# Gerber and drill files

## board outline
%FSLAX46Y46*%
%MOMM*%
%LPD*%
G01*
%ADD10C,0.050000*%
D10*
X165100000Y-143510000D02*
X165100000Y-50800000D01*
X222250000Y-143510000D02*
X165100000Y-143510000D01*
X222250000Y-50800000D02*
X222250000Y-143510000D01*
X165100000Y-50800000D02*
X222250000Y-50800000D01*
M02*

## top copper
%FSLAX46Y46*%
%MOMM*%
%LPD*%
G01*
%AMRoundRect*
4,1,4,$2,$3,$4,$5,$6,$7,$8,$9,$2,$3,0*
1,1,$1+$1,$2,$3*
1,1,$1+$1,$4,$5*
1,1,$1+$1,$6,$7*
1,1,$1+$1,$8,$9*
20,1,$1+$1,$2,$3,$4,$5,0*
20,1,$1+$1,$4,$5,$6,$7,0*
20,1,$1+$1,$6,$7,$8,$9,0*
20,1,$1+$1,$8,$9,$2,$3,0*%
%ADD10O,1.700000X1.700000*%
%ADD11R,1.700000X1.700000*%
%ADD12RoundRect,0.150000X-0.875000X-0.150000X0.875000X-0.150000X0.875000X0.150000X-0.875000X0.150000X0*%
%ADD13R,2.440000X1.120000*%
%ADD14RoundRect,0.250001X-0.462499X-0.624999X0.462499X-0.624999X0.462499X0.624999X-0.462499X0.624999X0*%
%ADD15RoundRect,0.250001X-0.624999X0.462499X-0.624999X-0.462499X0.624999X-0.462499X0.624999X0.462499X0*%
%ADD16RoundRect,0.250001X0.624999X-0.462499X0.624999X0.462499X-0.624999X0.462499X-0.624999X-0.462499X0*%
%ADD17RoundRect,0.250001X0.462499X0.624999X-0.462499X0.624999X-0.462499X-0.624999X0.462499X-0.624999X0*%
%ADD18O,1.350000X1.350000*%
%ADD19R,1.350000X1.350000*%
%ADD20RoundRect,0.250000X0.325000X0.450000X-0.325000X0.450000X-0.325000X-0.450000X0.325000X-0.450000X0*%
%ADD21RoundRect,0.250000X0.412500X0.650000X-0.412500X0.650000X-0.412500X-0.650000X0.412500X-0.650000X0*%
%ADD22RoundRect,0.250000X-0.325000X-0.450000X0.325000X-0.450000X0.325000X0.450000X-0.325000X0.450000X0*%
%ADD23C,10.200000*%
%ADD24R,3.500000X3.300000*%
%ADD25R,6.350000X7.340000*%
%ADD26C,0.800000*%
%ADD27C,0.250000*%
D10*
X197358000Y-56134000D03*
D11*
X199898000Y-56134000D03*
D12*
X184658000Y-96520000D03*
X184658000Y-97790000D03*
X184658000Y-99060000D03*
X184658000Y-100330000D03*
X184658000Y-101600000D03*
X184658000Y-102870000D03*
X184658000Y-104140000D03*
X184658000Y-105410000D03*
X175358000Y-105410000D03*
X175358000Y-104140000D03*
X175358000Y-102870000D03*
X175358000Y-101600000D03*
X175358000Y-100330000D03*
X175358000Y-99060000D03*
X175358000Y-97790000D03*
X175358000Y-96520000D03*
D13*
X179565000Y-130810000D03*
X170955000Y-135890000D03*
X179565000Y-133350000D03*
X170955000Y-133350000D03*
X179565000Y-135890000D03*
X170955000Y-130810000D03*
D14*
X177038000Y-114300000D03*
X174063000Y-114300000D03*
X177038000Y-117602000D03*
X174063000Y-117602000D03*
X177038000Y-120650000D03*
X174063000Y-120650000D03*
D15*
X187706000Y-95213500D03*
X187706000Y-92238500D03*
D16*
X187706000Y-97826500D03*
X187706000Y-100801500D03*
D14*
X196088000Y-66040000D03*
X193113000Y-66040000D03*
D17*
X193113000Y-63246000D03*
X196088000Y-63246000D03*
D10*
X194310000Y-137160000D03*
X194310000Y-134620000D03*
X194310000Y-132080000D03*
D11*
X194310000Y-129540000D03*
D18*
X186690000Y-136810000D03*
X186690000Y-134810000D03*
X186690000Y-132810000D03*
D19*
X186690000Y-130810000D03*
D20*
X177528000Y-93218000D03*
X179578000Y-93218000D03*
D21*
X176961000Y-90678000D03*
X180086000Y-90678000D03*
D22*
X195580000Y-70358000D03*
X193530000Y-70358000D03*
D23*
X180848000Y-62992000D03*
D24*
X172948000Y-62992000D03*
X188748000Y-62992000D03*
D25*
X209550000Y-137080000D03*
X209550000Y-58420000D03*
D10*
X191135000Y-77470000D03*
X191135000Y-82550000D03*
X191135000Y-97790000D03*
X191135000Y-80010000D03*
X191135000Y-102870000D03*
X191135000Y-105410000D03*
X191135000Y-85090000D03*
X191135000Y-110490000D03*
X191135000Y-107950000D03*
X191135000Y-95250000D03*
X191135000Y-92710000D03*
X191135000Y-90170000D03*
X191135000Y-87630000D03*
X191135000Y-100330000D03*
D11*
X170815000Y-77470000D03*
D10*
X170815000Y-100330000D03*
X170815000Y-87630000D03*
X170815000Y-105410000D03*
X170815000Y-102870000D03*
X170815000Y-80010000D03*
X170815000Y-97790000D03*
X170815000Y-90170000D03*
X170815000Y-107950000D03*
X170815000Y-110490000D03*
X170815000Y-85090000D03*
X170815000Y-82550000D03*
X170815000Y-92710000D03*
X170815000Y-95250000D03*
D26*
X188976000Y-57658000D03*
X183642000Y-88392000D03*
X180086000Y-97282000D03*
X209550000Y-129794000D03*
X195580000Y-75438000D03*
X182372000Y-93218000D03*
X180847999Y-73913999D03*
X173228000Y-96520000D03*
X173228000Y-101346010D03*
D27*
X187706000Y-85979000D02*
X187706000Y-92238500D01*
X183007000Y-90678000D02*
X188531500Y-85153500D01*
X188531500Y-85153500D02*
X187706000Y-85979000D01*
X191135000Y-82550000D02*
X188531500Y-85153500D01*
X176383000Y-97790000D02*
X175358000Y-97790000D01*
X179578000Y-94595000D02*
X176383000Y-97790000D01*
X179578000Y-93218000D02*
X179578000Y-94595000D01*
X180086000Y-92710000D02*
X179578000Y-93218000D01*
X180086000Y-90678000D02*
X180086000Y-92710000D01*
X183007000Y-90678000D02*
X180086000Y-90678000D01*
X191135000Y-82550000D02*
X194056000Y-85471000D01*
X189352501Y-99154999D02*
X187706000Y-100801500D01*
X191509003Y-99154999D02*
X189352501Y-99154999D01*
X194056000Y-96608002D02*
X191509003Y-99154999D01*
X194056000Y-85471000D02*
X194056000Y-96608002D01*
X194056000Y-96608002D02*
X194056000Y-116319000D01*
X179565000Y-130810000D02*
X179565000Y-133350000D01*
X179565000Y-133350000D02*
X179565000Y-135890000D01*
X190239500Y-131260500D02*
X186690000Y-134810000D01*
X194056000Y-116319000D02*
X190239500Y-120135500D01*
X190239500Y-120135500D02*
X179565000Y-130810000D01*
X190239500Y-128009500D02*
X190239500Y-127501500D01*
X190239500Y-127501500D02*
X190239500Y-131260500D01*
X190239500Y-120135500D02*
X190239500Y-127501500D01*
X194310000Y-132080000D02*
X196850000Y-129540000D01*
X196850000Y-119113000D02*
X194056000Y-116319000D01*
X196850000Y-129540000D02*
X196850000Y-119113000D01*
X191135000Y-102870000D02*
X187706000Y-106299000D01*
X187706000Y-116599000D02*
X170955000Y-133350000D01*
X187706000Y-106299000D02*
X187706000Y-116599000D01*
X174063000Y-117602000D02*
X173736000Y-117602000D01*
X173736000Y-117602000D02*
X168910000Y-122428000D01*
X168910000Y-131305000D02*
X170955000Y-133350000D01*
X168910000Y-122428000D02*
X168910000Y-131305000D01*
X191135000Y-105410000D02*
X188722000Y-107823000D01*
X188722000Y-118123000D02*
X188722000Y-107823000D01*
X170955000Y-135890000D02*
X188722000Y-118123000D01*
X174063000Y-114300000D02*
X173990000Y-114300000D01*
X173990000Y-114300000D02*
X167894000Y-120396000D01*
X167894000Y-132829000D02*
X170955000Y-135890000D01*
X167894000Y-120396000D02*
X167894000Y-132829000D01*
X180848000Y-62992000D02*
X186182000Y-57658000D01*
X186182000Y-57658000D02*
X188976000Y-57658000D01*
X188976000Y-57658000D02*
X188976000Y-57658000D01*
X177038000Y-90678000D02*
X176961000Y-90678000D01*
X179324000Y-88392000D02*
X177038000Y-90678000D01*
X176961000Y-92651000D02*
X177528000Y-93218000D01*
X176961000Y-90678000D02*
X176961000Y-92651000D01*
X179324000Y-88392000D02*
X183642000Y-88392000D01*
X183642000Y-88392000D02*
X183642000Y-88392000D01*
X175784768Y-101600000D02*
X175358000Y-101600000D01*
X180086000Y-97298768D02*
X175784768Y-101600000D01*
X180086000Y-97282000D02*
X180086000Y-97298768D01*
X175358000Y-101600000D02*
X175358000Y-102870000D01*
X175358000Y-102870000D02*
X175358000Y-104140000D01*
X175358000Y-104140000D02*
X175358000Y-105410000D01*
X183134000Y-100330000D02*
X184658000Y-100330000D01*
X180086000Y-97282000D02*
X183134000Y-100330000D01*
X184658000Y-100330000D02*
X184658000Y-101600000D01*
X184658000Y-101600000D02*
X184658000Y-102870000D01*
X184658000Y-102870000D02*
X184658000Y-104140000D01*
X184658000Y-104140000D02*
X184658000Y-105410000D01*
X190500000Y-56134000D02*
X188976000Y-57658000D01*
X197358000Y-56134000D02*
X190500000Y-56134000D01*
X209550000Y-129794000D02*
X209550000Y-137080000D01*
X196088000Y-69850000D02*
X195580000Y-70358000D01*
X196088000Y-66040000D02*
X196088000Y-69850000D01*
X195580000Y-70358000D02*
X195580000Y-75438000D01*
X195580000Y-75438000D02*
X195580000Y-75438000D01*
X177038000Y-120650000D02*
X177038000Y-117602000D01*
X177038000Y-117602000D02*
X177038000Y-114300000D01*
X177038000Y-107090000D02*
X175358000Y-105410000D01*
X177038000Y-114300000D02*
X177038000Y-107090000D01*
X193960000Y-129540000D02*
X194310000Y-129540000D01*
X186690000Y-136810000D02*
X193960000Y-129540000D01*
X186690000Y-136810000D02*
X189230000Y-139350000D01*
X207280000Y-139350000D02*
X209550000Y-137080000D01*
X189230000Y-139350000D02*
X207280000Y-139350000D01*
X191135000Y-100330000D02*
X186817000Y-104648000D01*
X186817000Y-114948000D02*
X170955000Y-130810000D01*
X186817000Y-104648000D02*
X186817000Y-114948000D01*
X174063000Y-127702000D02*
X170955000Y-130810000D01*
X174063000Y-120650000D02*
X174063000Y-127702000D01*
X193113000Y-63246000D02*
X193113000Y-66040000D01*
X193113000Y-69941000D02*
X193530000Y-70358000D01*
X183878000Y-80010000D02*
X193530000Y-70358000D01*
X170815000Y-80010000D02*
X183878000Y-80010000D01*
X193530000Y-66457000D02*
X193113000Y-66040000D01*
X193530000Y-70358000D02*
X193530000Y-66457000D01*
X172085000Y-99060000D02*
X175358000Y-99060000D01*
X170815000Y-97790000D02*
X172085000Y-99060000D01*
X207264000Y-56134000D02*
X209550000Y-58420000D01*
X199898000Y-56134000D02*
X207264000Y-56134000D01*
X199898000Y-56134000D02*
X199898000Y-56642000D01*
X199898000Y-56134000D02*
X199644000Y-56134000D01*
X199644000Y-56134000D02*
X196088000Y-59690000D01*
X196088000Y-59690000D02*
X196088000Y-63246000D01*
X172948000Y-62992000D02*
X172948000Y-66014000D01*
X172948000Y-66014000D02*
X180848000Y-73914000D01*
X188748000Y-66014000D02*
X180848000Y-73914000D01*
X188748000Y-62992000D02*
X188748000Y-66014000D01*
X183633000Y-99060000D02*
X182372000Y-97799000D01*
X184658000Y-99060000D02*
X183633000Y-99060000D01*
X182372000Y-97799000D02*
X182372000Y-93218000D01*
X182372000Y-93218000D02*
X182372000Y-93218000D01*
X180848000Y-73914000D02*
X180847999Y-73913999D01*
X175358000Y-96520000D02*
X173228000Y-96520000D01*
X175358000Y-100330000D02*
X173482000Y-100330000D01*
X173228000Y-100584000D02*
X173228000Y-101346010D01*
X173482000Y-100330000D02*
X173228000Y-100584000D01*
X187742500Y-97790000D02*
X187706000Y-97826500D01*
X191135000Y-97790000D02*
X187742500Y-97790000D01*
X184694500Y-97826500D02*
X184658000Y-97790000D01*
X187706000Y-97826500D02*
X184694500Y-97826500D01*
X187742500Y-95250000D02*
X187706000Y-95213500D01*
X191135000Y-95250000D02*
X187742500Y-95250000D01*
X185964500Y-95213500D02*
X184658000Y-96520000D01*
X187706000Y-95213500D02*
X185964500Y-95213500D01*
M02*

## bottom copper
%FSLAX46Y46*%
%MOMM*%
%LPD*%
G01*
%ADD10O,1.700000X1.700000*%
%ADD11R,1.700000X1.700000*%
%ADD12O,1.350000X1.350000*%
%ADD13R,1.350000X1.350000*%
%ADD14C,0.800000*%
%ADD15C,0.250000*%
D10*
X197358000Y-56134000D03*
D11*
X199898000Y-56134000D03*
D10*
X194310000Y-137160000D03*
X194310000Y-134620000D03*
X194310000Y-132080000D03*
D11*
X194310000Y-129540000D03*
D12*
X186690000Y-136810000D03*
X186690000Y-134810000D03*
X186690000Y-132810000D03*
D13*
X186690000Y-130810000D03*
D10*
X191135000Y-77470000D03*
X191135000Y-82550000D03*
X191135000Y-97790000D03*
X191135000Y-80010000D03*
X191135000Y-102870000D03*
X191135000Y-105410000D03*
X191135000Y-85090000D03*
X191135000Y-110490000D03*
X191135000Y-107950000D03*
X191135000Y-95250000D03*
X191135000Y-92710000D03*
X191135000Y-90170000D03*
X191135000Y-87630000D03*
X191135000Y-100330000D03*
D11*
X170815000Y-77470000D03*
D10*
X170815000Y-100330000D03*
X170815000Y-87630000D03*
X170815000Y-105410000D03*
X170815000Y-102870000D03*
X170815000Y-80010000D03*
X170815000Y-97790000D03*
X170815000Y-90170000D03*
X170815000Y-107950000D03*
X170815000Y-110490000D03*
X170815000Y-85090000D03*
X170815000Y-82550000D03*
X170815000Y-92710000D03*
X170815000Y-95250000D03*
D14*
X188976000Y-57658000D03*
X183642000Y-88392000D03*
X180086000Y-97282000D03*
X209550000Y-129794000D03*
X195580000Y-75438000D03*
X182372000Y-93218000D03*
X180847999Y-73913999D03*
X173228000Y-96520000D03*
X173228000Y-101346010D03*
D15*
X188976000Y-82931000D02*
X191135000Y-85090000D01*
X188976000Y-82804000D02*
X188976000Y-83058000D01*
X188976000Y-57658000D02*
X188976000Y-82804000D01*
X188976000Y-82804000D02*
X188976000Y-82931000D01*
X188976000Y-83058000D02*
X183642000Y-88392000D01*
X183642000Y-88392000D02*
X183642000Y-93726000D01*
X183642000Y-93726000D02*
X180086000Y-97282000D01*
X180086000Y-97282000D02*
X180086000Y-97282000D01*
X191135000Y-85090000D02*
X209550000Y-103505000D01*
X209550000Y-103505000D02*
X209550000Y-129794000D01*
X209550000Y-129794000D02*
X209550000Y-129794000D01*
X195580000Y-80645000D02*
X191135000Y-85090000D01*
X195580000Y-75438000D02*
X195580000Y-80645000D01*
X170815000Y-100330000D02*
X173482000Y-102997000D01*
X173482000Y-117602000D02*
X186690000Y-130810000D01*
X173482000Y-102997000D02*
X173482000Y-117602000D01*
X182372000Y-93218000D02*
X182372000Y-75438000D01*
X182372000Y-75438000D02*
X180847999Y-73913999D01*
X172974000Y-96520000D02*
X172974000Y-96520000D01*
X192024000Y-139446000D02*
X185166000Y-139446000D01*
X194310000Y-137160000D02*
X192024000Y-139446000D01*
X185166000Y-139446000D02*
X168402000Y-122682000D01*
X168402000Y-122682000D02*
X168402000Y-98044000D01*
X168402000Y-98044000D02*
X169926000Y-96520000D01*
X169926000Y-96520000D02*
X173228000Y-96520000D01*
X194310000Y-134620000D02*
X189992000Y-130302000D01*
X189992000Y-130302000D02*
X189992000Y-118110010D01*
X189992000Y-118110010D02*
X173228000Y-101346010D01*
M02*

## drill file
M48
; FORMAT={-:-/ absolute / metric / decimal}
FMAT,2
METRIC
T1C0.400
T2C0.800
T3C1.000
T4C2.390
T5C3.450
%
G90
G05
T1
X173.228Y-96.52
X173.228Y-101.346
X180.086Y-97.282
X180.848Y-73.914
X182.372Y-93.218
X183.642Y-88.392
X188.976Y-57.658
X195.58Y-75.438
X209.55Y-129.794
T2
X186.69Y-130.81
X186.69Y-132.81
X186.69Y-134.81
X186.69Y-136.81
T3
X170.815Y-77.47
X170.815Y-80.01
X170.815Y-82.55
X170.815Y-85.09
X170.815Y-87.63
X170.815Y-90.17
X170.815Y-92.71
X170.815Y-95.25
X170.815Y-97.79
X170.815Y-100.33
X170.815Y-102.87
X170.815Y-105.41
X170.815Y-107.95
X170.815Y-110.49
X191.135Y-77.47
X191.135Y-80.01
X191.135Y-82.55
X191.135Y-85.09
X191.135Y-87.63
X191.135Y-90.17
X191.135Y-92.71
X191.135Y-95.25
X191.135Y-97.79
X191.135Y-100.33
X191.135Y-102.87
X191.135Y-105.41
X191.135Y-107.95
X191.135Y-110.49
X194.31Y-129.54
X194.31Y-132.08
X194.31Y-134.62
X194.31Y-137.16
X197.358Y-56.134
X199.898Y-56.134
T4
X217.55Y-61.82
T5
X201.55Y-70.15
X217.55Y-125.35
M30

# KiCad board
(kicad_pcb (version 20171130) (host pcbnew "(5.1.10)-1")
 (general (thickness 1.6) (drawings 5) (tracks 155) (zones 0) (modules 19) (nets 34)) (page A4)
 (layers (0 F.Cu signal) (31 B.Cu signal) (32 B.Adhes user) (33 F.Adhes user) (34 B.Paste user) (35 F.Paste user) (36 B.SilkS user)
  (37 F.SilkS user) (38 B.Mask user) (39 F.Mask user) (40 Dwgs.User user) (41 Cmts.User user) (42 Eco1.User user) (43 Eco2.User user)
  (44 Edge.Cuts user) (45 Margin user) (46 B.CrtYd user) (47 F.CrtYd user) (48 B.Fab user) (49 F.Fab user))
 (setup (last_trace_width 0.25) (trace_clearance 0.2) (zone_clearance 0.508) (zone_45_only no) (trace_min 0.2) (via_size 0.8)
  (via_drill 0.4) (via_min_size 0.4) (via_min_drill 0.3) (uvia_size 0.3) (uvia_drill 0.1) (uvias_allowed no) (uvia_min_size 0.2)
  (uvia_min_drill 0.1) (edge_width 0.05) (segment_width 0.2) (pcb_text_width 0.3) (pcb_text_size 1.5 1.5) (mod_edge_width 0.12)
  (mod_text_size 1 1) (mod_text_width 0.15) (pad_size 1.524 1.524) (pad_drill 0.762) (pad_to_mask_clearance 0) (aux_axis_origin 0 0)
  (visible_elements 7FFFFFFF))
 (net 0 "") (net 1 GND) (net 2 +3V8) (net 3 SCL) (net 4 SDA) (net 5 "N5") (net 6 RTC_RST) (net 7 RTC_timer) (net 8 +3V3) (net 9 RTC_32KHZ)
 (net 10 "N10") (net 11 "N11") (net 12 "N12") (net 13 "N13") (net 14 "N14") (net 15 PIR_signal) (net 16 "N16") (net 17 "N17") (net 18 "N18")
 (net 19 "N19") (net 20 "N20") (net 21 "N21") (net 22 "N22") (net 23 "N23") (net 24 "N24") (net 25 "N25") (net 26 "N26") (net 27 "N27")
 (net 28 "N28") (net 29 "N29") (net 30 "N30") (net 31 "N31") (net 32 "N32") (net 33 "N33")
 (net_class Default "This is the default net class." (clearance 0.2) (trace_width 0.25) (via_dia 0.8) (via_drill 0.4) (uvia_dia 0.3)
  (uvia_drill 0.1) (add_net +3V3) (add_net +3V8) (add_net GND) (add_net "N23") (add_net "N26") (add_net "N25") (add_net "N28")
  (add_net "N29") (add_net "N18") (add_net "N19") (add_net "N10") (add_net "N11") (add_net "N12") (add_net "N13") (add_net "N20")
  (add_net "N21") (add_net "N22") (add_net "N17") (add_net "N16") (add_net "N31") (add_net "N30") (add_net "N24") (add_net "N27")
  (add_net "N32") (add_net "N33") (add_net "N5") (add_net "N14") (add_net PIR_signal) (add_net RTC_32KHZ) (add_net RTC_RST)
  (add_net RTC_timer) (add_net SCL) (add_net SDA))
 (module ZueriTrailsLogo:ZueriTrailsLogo (layer B.Cu) (at 201.93 96.52 270)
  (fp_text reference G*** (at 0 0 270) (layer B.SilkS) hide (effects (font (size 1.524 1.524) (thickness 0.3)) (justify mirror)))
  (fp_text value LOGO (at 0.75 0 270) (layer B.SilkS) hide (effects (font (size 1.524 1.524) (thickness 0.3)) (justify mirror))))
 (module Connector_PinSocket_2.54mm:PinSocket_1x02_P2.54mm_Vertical (layer F.Cu) (at 199.898 56.134 270)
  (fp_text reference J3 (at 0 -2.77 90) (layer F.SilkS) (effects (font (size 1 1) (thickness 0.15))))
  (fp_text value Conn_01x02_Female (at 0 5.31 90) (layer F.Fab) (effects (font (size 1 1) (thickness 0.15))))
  (pad 2 thru_hole oval (at 0 2.54 270) (size 1.7 1.7) (drill 1) (layers *.Cu *.Mask) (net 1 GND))
  (pad 1 thru_hole rect (at 0 0 270) (size 1.7 1.7) (drill 1) (layers *.Cu *.Mask) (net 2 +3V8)))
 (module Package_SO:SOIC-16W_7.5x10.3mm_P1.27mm (layer F.Cu) (at 180.008 100.965)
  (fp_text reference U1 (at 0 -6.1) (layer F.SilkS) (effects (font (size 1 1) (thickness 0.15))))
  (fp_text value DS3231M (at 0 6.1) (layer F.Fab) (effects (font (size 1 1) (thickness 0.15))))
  (pad 16 smd roundrect (at 4.65 -4.445) (size 2.05 0.6) (layers F.Cu F.Paste F.Mask) (roundrect_rratio 0.25) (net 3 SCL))
  (pad 15 smd roundrect (at 4.65 -3.175) (size 2.05 0.6) (layers F.Cu F.Paste F.Mask) (roundrect_rratio 0.25) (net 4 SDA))
  (pad 14 smd roundrect (at 4.65 -1.905) (size 2.05 0.6) (layers F.Cu F.Paste F.Mask) (roundrect_rratio 0.25) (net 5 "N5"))
  (pad 13 smd roundrect (at 4.65 -0.635) (size 2.05 0.6) (layers F.Cu F.Paste F.Mask) (roundrect_rratio 0.25) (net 1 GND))
  (pad 12 smd roundrect (at 4.65 0.635) (size 2.05 0.6) (layers F.Cu F.Paste F.Mask) (roundrect_rratio 0.25) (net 1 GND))
  (pad 11 smd roundrect (at 4.65 1.905) (size 2.05 0.6) (layers F.Cu F.Paste F.Mask) (roundrect_rratio 0.25) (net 1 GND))
  (pad 10 smd roundrect (at 4.65 3.175) (size 2.05 0.6) (layers F.Cu F.Paste F.Mask) (roundrect_rratio 0.25) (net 1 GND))
  (pad 9 smd roundrect (at 4.65 4.445) (size 2.05 0.6) (layers F.Cu F.Paste F.Mask) (roundrect_rratio 0.25) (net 1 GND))
  (pad 8 smd roundrect (at -4.65 4.445) (size 2.05 0.6) (layers F.Cu F.Paste F.Mask) (roundrect_rratio 0.25) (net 1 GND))
  (pad 7 smd roundrect (at -4.65 3.175) (size 2.05 0.6) (layers F.Cu F.Paste F.Mask) (roundrect_rratio 0.25) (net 1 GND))
  (pad 6 smd roundrect (at -4.65 1.905) (size 2.05 0.6) (layers F.Cu F.Paste F.Mask) (roundrect_rratio 0.25) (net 1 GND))
  (pad 5 smd roundrect (at -4.65 0.635) (size 2.05 0.6) (layers F.Cu F.Paste F.Mask) (roundrect_rratio 0.25) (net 1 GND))
  (pad 4 smd roundrect (at -4.65 -0.635) (size 2.05 0.6) (layers F.Cu F.Paste F.Mask) (roundrect_rratio 0.25) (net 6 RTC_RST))
  (pad 3 smd roundrect (at -4.65 -1.905) (size 2.05 0.6) (layers F.Cu F.Paste F.Mask) (roundrect_rratio 0.25) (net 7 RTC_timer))
  (pad 2 smd roundrect (at -4.65 -3.175) (size 2.05 0.6) (layers F.Cu F.Paste F.Mask) (roundrect_rratio 0.25) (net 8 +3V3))
  (pad 1 smd roundrect (at -4.65 -4.445) (size 2.05 0.6) (layers F.Cu F.Paste F.Mask) (roundrect_rratio 0.25) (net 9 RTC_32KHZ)))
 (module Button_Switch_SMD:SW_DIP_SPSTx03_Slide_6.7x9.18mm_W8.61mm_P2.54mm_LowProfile (layer F.Cu) (at 175.26 133.35)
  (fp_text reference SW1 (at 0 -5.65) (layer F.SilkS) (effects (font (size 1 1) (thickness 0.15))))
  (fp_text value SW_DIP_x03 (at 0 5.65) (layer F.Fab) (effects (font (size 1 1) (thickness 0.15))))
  (pad 6 smd rect (at 4.305 -2.54) (size 2.44 1.12) (layers F.Cu F.Paste F.Mask) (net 8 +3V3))
  (pad 3 smd rect (at -4.305 2.54) (size 2.44 1.12) (layers F.Cu F.Paste F.Mask) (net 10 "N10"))
  (pad 5 smd rect (at 4.305 0) (size 2.44 1.12) (layers F.Cu F.Paste F.Mask) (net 8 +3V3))
  (pad 2 smd rect (at -4.305 0) (size 2.44 1.12) (layers F.Cu F.Paste F.Mask) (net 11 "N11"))
  (pad 4 smd rect (at 4.305 2.54) (size 2.44 1.12) (layers F.Cu F.Paste F.Mask) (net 8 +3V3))
  (pad 1 smd rect (at -4.305 -2.54) (size 2.44 1.12) (layers F.Cu F.Paste F.Mask) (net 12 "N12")))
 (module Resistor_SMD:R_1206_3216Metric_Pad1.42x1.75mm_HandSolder (layer F.Cu) (at 175.5505 114.3)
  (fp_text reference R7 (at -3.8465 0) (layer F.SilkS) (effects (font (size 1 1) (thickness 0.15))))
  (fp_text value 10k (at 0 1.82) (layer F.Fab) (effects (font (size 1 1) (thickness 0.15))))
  (pad 2 smd roundrect (at 1.4875 0) (size 1.425 1.75) (layers F.Cu F.Paste F.Mask) (roundrect_rratio 0.175439) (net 1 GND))
  (pad 1 smd roundrect (at -1.4875 0) (size 1.425 1.75) (layers F.Cu F.Paste F.Mask) (roundrect_rratio 0.175439) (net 10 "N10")))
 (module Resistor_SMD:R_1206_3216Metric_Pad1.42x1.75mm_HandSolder (layer F.Cu) (at 175.5505 117.602)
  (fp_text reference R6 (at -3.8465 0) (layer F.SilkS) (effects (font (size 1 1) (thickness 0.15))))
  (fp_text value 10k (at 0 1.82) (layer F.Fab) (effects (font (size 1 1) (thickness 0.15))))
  (pad 2 smd roundrect (at 1.4875 0) (size 1.425 1.75) (layers F.Cu F.Paste F.Mask) (roundrect_rratio 0.175439) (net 1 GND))
  (pad 1 smd roundrect (at -1.4875 0) (size 1.425 1.75) (layers F.Cu F.Paste F.Mask) (roundrect_rratio 0.175439) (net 11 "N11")))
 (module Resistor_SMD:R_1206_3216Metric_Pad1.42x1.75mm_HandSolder (layer F.Cu) (at 175.5505 120.65)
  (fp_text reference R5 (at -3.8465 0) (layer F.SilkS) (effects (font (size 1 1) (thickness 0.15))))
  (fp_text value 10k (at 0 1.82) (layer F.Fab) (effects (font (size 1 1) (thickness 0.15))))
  (pad 2 smd roundrect (at 1.4875 0) (size 1.425 1.75) (layers F.Cu F.Paste F.Mask) (roundrect_rratio 0.175439) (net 1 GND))
  (pad 1 smd roundrect (at -1.4875 0) (size 1.425 1.75) (layers F.Cu F.Paste F.Mask) (roundrect_rratio 0.175439) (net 12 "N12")))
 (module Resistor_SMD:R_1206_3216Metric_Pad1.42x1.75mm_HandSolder (layer F.Cu) (at 187.706 93.726 270)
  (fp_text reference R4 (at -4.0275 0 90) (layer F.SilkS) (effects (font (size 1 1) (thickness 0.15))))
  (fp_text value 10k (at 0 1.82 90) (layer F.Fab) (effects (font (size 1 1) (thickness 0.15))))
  (pad 2 smd roundrect (at 1.4875 0 270) (size 1.425 1.75) (layers F.Cu F.Paste F.Mask) (roundrect_rratio 0.175439) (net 3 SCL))
  (pad 1 smd roundrect (at -1.4875 0 270) (size 1.425 1.75) (layers F.Cu F.Paste F.Mask) (roundrect_rratio 0.175439) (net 8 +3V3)))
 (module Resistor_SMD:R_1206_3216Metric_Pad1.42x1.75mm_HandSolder (layer F.Cu) (at 187.706 99.314 90)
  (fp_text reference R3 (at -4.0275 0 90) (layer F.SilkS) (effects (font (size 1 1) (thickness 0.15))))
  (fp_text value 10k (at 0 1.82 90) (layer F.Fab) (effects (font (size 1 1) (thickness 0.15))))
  (pad 2 smd roundrect (at 1.4875 0 90) (size 1.425 1.75) (layers F.Cu F.Paste F.Mask) (roundrect_rratio 0.175439) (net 4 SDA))
  (pad 1 smd roundrect (at -1.4875 0 90) (size 1.425 1.75) (layers F.Cu F.Paste F.Mask) (roundrect_rratio 0.175439) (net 8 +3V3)))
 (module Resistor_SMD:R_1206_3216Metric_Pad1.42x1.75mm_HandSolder (layer F.Cu) (at 194.6005 66.04)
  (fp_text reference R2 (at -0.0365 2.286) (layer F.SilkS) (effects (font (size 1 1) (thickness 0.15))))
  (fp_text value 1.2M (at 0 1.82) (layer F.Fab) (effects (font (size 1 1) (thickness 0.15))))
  (pad 2 smd roundrect (at 1.4875 0) (size 1.425 1.75) (layers F.Cu F.Paste F.Mask) (roundrect_rratio 0.175439) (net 1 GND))
  (pad 1 smd roundrect (at -1.4875 0) (size 1.425 1.75) (layers F.Cu F.Paste F.Mask) (roundrect_rratio 0.175439) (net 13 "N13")))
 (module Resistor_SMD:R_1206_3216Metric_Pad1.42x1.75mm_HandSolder (layer F.Cu) (at 194.6005 63.246 180)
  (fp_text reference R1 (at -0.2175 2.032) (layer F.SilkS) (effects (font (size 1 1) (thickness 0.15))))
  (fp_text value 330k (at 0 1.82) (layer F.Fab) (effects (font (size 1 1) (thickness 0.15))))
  (pad 2 smd roundrect (at 1.4875 0 180) (size 1.425 1.75) (layers F.Cu F.Paste F.Mask) (roundrect_rratio 0.175439) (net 13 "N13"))
  (pad 1 smd roundrect (at -1.4875 0 180) (size 1.425 1.75) (layers F.Cu F.Paste F.Mask) (roundrect_rratio 0.175439) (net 2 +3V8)))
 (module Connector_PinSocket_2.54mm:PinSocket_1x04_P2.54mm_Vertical (layer F.Cu) (at 194.31 129.54)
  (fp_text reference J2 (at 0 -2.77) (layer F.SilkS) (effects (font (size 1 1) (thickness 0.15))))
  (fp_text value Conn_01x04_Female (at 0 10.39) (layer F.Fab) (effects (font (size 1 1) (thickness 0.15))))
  (pad 4 thru_hole oval (at 0 7.62) (size 1.7 1.7) (drill 1) (layers *.Cu *.Mask) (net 9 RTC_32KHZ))
  (pad 3 thru_hole oval (at 0 5.08) (size 1.7 1.7) (drill 1) (layers *.Cu *.Mask) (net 6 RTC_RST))
  (pad 2 thru_hole oval (at 0 2.54) (size 1.7 1.7) (drill 1) (layers *.Cu *.Mask) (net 8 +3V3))
  (pad 1 thru_hole rect (at 0 0) (size 1.7 1.7) (drill 1) (layers *.Cu *.Mask) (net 1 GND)))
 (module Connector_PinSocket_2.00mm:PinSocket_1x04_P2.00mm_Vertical (layer F.Cu) (at 186.69 130.81)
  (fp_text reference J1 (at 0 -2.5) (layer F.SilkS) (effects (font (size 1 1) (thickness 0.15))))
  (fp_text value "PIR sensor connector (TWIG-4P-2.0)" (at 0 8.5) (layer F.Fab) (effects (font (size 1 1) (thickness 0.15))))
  (pad 4 thru_hole oval (at 0 6) (size 1.35 1.35) (drill 0.8) (layers *.Cu *.Mask) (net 1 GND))
  (pad 3 thru_hole oval (at 0 4) (size 1.35 1.35) (drill 0.8) (layers *.Cu *.Mask) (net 8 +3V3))
  (pad 2 thru_hole oval (at 0 2) (size 1.35 1.35) (drill 0.8) (layers *.Cu *.Mask) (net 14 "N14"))
  (pad 1 thru_hole rect (at 0 0) (size 1.35 1.35) (drill 0.8) (layers *.Cu *.Mask) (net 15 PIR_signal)))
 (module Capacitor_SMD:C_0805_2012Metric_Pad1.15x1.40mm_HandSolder (layer F.Cu) (at 178.553 93.218 180)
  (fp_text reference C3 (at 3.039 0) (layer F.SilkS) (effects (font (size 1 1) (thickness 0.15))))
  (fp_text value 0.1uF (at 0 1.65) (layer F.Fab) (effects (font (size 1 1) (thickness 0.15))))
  (pad 2 smd roundrect (at 1.025 0 180) (size 1.15 1.4) (layers F.Cu F.Paste F.Mask) (roundrect_rratio 0.217391) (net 1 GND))
  (pad 1 smd roundrect (at -1.025 0 180) (size 1.15 1.4) (layers F.Cu F.Paste F.Mask) (roundrect_rratio 0.217391) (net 8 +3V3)))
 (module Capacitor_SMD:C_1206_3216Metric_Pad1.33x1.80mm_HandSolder (layer F.Cu) (at 178.5235 90.678 180)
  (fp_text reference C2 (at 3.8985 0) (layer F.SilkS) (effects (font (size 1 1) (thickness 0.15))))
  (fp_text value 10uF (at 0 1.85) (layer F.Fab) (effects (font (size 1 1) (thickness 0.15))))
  (pad 2 smd roundrect (at 1.5625 0 180) (size 1.325 1.8) (layers F.Cu F.Paste F.Mask) (roundrect_rratio 0.188679) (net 1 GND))
  (pad 1 smd roundrect (at -1.5625 0 180) (size 1.325 1.8) (layers F.Cu F.Paste F.Mask) (roundrect_rratio 0.188679) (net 8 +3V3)))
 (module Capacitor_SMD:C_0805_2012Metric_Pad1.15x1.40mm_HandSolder (layer F.Cu) (at 194.555 70.358)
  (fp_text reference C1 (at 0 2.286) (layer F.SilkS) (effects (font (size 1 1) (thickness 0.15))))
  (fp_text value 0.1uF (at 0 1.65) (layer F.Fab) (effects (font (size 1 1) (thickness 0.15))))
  (pad 2 smd roundrect (at 1.025 0) (size 1.15 1.4) (layers F.Cu F.Paste F.Mask) (roundrect_rratio 0.217391) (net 1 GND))
  (pad 1 smd roundrect (at -1.025 0) (size 1.15 1.4) (layers F.Cu F.Paste F.Mask) (roundrect_rratio 0.217391) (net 13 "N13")))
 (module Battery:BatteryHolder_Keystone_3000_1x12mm (layer F.Cu) (at 180.848 62.992 180)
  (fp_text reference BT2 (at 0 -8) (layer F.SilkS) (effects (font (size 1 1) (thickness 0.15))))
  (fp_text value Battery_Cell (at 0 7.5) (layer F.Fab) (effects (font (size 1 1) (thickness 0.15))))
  (pad 2 smd circle (at 0 0 180) (size 10.2 10.2) (layers F.Cu F.Mask) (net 1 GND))
  (pad 1 smd rect (at 7.9 0 180) (size 3.5 3.3) (layers F.Cu F.Paste F.Mask) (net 5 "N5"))
  (pad 1 smd rect (at -7.9 0 180) (size 3.5 3.3) (layers F.Cu F.Paste F.Mask) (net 5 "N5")))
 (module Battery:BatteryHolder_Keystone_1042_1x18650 (layer F.Cu) (at 209.55 97.75 270)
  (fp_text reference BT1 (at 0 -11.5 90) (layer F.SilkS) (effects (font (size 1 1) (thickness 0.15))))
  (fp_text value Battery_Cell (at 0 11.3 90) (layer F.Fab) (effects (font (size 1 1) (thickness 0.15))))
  (pad "" np_thru_hole circle (at -35.93 -8 270) (size 2.39 2.39) (drill 2.39) (layers *.Cu *.Mask))
  (pad "" np_thru_hole circle (at -27.6 8 270) (size 3.45 3.45) (drill 3.45) (layers *.Cu *.Mask))
  (pad "" np_thru_hole circle (at 27.6 -8 270) (size 3.45 3.45) (drill 3.45) (layers *.Cu *.Mask))
  (pad 2 smd rect (at 39.33 0 270) (size 7.34 6.35) (layers F.Cu F.Paste F.Mask) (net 1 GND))
  (pad 1 smd rect (at -39.33 0 270) (size 7.34 6.35) (layers F.Cu F.Paste F.Mask) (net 2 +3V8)))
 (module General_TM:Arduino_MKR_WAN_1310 (layer F.Cu) (at 170.815 77.47)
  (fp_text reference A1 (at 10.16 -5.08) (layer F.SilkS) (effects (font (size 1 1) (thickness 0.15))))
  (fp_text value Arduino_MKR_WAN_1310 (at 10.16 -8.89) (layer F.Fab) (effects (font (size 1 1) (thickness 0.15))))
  (pad 28 thru_hole oval (at 20.32 0) (size 1.7 1.7) (drill 1) (layers *.Cu *.Mask) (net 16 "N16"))
  (pad 26 thru_hole oval (at 20.32 5.08) (size 1.7 1.7) (drill 1) (layers *.Cu *.Mask) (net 8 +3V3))
  (pad 20 thru_hole oval (at 20.32 20.32) (size 1.7 1.7) (drill 1) (layers *.Cu *.Mask) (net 4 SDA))
  (pad 27 thru_hole oval (at 20.32 2.54) (size 1.7 1.7) (drill 1) (layers *.Cu *.Mask) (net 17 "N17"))
  (pad 18 thru_hole oval (at 20.32 25.4) (size 1.7 1.7) (drill 1) (layers *.Cu *.Mask) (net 11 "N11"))
  (pad 17 thru_hole oval (at 20.32 27.94) (size 1.7 1.7) (drill 1) (layers *.Cu *.Mask) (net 10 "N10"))
  (pad 25 thru_hole oval (at 20.32 7.62) (size 1.7 1.7) (drill 1) (layers *.Cu *.Mask) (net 1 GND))
  (pad 15 thru_hole oval (at 20.32 33.02) (size 1.7 1.7) (drill 1) (layers *.Cu *.Mask) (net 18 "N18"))
  (pad 16 thru_hole oval (at 20.32 30.48) (size 1.7 1.7) (drill 1) (layers *.Cu *.Mask) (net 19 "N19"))
  (pad 21 thru_hole oval (at 20.32 17.78) (size 1.7 1.7) (drill 1) (layers *.Cu *.Mask) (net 3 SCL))
  (pad 22 thru_hole oval (at 20.32 15.24) (size 1.7 1.7) (drill 1) (layers *.Cu *.Mask) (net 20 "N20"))
  (pad 23 thru_hole oval (at 20.32 12.7) (size 1.7 1.7) (drill 1) (layers *.Cu *.Mask) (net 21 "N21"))
  (pad 24 thru_hole oval (at 20.32 10.16) (size 1.7 1.7) (drill 1) (layers *.Cu *.Mask) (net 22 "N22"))
  (pad 19 thru_hole oval (at 20.32 22.86) (size 1.7 1.7) (drill 1) (layers *.Cu *.Mask) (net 12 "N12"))
  (pad 1 thru_hole rect (at 0 0) (size 1.7 1.7) (drill 1) (layers *.Cu *.Mask) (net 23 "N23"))
  (pad 10 thru_hole oval (at 0 22.86) (size 1.7 1.7) (drill 1) (layers *.Cu *.Mask) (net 15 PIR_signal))
  (pad 5 thru_hole oval (at 0 10.16) (size 1.7 1.7) (drill 1) (layers *.Cu *.Mask) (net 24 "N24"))
  (pad 12 thru_hole oval (at 0 27.94) (size 1.7 1.7) (drill 1) (layers *.Cu *.Mask) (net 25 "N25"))
  (pad 11 thru_hole oval (at 0 25.4) (size 1.7 1.7) (drill 1) (layers *.Cu *.Mask) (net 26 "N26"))
  (pad 2 thru_hole oval (at 0 2.54) (size 1.7 1.7) (drill 1) (layers *.Cu *.Mask) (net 13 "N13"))
  (pad 9 thru_hole oval (at 0 20.32) (size 1.7 1.7) (drill 1) (layers *.Cu *.Mask) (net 7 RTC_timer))
  (pad 6 thru_hole oval (at 0 12.7) (size 1.7 1.7) (drill 1) (layers *.Cu *.Mask) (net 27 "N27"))
  (pad 13 thru_hole oval (at 0 30.48) (size 1.7 1.7) (drill 1) (layers *.Cu *.Mask) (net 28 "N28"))
  (pad 14 thru_hole oval (at 0 33.02) (size 1.7 1.7) (drill 1) (layers *.Cu *.Mask) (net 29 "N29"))
  (pad 4 thru_hole oval (at 0 7.62) (size 1.7 1.7) (drill 1) (layers *.Cu *.Mask) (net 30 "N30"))
  (pad 3 thru_hole oval (at 0 5.08) (size 1.7 1.7) (drill 1) (layers *.Cu *.Mask) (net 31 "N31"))
  (pad 7 thru_hole oval (at 0 15.24) (size 1.7 1.7) (drill 1) (layers *.Cu *.Mask) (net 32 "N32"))
  (pad 8 thru_hole oval (at 0 17.78) (size 1.7 1.7) (drill 1) (layers *.Cu *.Mask) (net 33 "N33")))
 (gr_line (start 165.1 143.51) (end 165.1 50.8) (layer Edge.Cuts) (width 0.05))
 (gr_line (start 222.25 143.51) (end 165.1 143.51) (layer Edge.Cuts) (width 0.05))
 (gr_line (start 222.25 50.8) (end 222.25 143.51) (layer Edge.Cuts) (width 0.05))
 (gr_line (start 165.1 50.8) (end 222.25 50.8) (layer Edge.Cuts) (width 0.05))
 (segment (start 187.706 85.979) (end 187.706 92.2385) (width 0.25) (layer F.Cu) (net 8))
 (segment (start 183.007 90.678) (end 188.5315 85.1535) (width 0.25) (layer F.Cu) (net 8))
 (segment (start 188.5315 85.1535) (end 187.706 85.979) (width 0.25) (layer F.Cu) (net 8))
 (segment (start 191.135 82.55) (end 188.5315 85.1535) (width 0.25) (layer F.Cu) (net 8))
 (segment (start 176.383 97.79) (end 175.358 97.79) (width 0.25) (layer F.Cu) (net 8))
 (segment (start 179.578 94.595) (end 176.383 97.79) (width 0.25) (layer F.Cu) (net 8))
 (segment (start 179.578 93.218) (end 179.578 94.595) (width 0.25) (layer F.Cu) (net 8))
 (segment (start 180.086 92.71) (end 179.578 93.218) (width 0.25) (layer F.Cu) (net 8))
 (segment (start 180.086 90.678) (end 180.086 92.71) (width 0.25) (layer F.Cu) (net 8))
 (segment (start 183.007 90.678) (end 180.086 90.678) (width 0.25) (layer F.Cu) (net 8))
 (segment (start 191.135 82.55) (end 194.056 85.471) (width 0.25) (layer F.Cu) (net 8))
 (segment (start 189.352501 99.154999) (end 187.706 100.8015) (width 0.25) (layer F.Cu) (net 8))
 (segment (start 191.509003 99.154999) (end 189.352501 99.154999) (width 0.25) (layer F.Cu) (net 8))
 (segment (start 194.056 96.608002) (end 191.509003 99.154999) (width 0.25) (layer F.Cu) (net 8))
 (segment (start 194.056 85.471) (end 194.056 96.608002) (width 0.25) (layer F.Cu) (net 8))
 (segment (start 194.056 96.608002) (end 194.056 116.319) (width 0.25) (layer F.Cu) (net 8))
 (segment (start 179.565 130.81) (end 179.565 133.35) (width 0.25) (layer F.Cu) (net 8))
 (segment (start 179.565 133.35) (end 179.565 135.89) (width 0.25) (layer F.Cu) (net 8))
 (segment (start 190.2395 131.2605) (end 186.69 134.81) (width 0.25) (layer F.Cu) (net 8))
 (segment (start 194.056 116.319) (end 190.2395 120.1355) (width 0.25) (layer F.Cu) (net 8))
 (segment (start 190.2395 120.1355) (end 179.565 130.81) (width 0.25) (layer F.Cu) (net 8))
 (segment (start 190.2395 128.0095) (end 190.2395 127.5015) (width 0.25) (layer F.Cu) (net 8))
 (segment (start 190.2395 127.5015) (end 190.2395 131.2605) (width 0.25) (layer F.Cu) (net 8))
 (segment (start 190.2395 120.1355) (end 190.2395 127.5015) (width 0.25) (layer F.Cu) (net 8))
 (segment (start 194.31 132.08) (end 196.85 129.54) (width 0.25) (layer F.Cu) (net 8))
 (segment (start 196.85 119.113) (end 194.056 116.319) (width 0.25) (layer F.Cu) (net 8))
 (segment (start 196.85 129.54) (end 196.85 119.113) (width 0.25) (layer F.Cu) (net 8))
 (segment (start 191.135 102.87) (end 187.706 106.299) (width 0.25) (layer F.Cu) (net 11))
 (segment (start 187.706 116.599) (end 170.955 133.35) (width 0.25) (layer F.Cu) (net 11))
 (segment (start 187.706 106.299) (end 187.706 116.599) (width 0.25) (layer F.Cu) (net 11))
 (segment (start 174.063 117.602) (end 173.736 117.602) (width 0.25) (layer F.Cu) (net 11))
 (segment (start 173.736 117.602) (end 168.91 122.428) (width 0.25) (layer F.Cu) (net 11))
 (segment (start 168.91 131.305) (end 170.955 133.35) (width 0.25) (layer F.Cu) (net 11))
 (segment (start 168.91 122.428) (end 168.91 131.305) (width 0.25) (layer F.Cu) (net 11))
 (segment (start 191.135 105.41) (end 188.722 107.823) (width 0.25) (layer F.Cu) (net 10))
 (segment (start 188.722 118.123) (end 188.722 107.823) (width 0.25) (layer F.Cu) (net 10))
 (segment (start 170.955 135.89) (end 188.722 118.123) (width 0.25) (layer F.Cu) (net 10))
 (segment (start 174.063 114.3) (end 173.99 114.3) (width 0.25) (layer F.Cu) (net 10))
 (segment (start 173.99 114.3) (end 167.894 120.396) (width 0.25) (layer F.Cu) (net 10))
 (segment (start 167.894 132.829) (end 170.955 135.89) (width 0.25) (layer F.Cu) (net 10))
 (segment (start 167.894 120.396) (end 167.894 132.829) (width 0.25) (layer F.Cu) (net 10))
 (segment (start 180.848 62.992) (end 186.182 57.658) (width 0.25) (layer F.Cu) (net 1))
 (segment (start 186.182 57.658) (end 188.976 57.658) (width 0.25) (layer F.Cu) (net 1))
 (segment (start 188.976 57.658) (end 188.976 57.658) (width 0.25) (layer F.Cu) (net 1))
 (via (at 188.976 57.658) (size 0.8) (drill 0.4) (layers F.Cu B.Cu) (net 1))
 (segment (start 188.976 82.931) (end 191.135 85.09) (width 0.25) (layer B.Cu) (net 1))
 (segment (start 188.976 82.804) (end 188.976 83.058) (width 0.25) (layer B.Cu) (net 1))
 (segment (start 188.976 57.658) (end 188.976 82.804) (width 0.25) (layer B.Cu) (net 1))
 (segment (start 188.976 82.804) (end 188.976 82.931) (width 0.25) (layer B.Cu) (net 1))
 (segment (start 188.976 83.058) (end 183.642 88.392) (width 0.25) (layer B.Cu) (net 1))
 (segment (start 177.038 90.678) (end 176.961 90.678) (width 0.25) (layer F.Cu) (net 1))
 (segment (start 179.324 88.392) (end 177.038 90.678) (width 0.25) (layer F.Cu) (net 1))
 (segment (start 176.961 92.651) (end 177.528 93.218) (width 0.25) (layer F.Cu) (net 1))
 (segment (start 176.961 90.678) (end 176.961 92.651) (width 0.25) (layer F.Cu) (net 1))
 (segment (start 179.324 88.392) (end 183.642 88.392) (width 0.25) (layer F.Cu) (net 1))
 (segment (start 183.642 88.392) (end 183.642 88.392) (width 0.25) (layer F.Cu) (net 1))
 (via (at 183.642 88.392) (size 0.8) (drill 0.4) (layers F.Cu B.Cu) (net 1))
 (segment (start 183.642 88.392) (end 183.642 93.726) (width 0.25) (layer B.Cu) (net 1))
 (segment (start 183.642 93.726) (end 180.086 97.282) (width 0.25) (layer B.Cu) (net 1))
 (segment (start 180.086 97.282) (end 180.086 97.282) (width 0.25) (layer B.Cu) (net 1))
 (via (at 180.086 97.282) (size 0.8) (drill 0.4) (layers F.Cu B.Cu) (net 1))
 (segment (start 175.784768 101.6) (end 175.358 101.6) (width 0.25) (layer F.Cu) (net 1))
 (segment (start 180.086 97.298768) (end 175.784768 101.6) (width 0.25) (layer F.Cu) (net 1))
 (segment (start 180.086 97.282) (end 180.086 97.298768) (width 0.25) (layer F.Cu) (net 1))
 (segment (start 175.358 101.6) (end 175.358 102.87) (width 0.25) (layer F.Cu) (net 1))
 (segment (start 175.358 102.87) (end 175.358 104.14) (width 0.25) (layer F.Cu) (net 1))
 (segment (start 175.358 104.14) (end 175.358 105.41) (width 0.25) (layer F.Cu) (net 1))
 (segment (start 183.134 100.33) (end 184.658 100.33) (width 0.25) (layer F.Cu) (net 1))
 (segment (start 180.086 97.282) (end 183.134 100.33) (width 0.25) (layer F.Cu) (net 1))
 (segment (start 184.658 100.33) (end 184.658 101.6) (width 0.25) (layer F.Cu) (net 1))
 (segment (start 184.658 101.6) (end 184.658 102.87) (width 0.25) (layer F.Cu) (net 1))
 (segment (start 184.658 102.87) (end 184.658 104.14) (width 0.25) (layer F.Cu) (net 1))
 (segment (start 184.658 104.14) (end 184.658 105.41) (width 0.25) (layer F.Cu) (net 1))
 (segment (start 190.5 56.134) (end 188.976 57.658) (width 0.25) (layer F.Cu) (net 1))
 (segment (start 197.358 56.134) (end 190.5 56.134) (width 0.25) (layer F.Cu) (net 1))
 (segment (start 191.135 85.09) (end 209.55 103.505) (width 0.25) (layer B.Cu) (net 1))
 (segment (start 209.55 103.505) (end 209.55 129.794) (width 0.25) (layer B.Cu) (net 1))
 (segment (start 209.55 129.794) (end 209.55 129.794) (width 0.25) (layer B.Cu) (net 1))
 (via (at 209.55 129.794) (size 0.8) (drill 0.4) (layers F.Cu B.Cu) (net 1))
 (segment (start 209.55 129.794) (end 209.55 137.08) (width 0.25) (layer F.Cu) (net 1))
 (segment (start 196.088 69.85) (end 195.58 70.358) (width 0.25) (layer F.Cu) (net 1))
 (segment (start 196.088 66.04) (end 196.088 69.85) (width 0.25) (layer F.Cu) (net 1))
 (segment (start 195.58 70.358) (end 195.58 75.438) (width 0.25) (layer F.Cu) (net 1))
 (segment (start 195.58 75.438) (end 195.58 75.438) (width 0.25) (layer F.Cu) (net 1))
 (via (at 195.58 75.438) (size 0.8) (drill 0.4) (layers F.Cu B.Cu) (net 1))
 (segment (start 195.58 80.645) (end 191.135 85.09) (width 0.25) (layer B.Cu) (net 1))
 (segment (start 195.58 75.438) (end 195.58 80.645) (width 0.25) (layer B.Cu) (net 1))
 (segment (start 177.038 120.65) (end 177.038 117.602) (width 0.25) (layer F.Cu) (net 1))
 (segment (start 177.038 117.602) (end 177.038 114.3) (width 0.25) (layer F.Cu) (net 1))
 (segment (start 177.038 107.09) (end 175.358 105.41) (width 0.25) (layer F.Cu) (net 1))
 (segment (start 177.038 114.3) (end 177.038 107.09) (width 0.25) (layer F.Cu) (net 1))
 (segment (start 193.96 129.54) (end 194.31 129.54) (width 0.25) (layer F.Cu) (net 1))
 (segment (start 186.69 136.81) (end 193.96 129.54) (width 0.25) (layer F.Cu) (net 1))
 (segment (start 186.69 136.81) (end 189.23 139.35) (width 0.25) (layer F.Cu) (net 1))
 (segment (start 207.28 139.35) (end 209.55 137.08) (width 0.25) (layer F.Cu) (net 1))
 (segment (start 189.23 139.35) (end 207.28 139.35) (width 0.25) (layer F.Cu) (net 1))
 (segment (start 191.135 100.33) (end 186.817 104.648) (width 0.25) (layer F.Cu) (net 12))
 (segment (start 186.817 114.948) (end 170.955 130.81) (width 0.25) (layer F.Cu) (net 12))
 (segment (start 186.817 104.648) (end 186.817 114.948) (width 0.25) (layer F.Cu) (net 12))
 (segment (start 174.063 127.702) (end 170.955 130.81) (width 0.25) (layer F.Cu) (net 12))
 (segment (start 174.063 120.65) (end 174.063 127.702) (width 0.25) (layer F.Cu) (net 12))
 (segment (start 170.815 100.33) (end 173.482 102.997) (width 0.25) (layer B.Cu) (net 15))
 (segment (start 173.482 117.602) (end 186.69 130.81) (width 0.25) (layer B.Cu) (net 15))
 (segment (start 173.482 102.997) (end 173.482 117.602) (width 0.25) (layer B.Cu) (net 15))
 (segment (start 193.113 63.246) (end 193.113 66.04) (width 0.25) (layer F.Cu) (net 13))
 (segment (start 193.113 69.941) (end 193.53 70.358) (width 0.25) (layer F.Cu) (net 13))
 (segment (start 183.878 80.01) (end 193.53 70.358) (width 0.25) (layer F.Cu) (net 13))
 (segment (start 170.815 80.01) (end 183.878 80.01) (width 0.25) (layer F.Cu) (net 13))
 (segment (start 193.53 66.457) (end 193.113 66.04) (width 0.25) (layer F.Cu) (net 13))
 (segment (start 193.53 70.358) (end 193.53 66.457) (width 0.25) (layer F.Cu) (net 13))
 (segment (start 172.085 99.06) (end 175.358 99.06) (width 0.25) (layer F.Cu) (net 7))
 (segment (start 170.815 97.79) (end 172.085 99.06) (width 0.25) (layer F.Cu) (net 7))
 (segment (start 207.264 56.134) (end 209.55 58.42) (width 0.25) (layer F.Cu) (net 2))
 (segment (start 199.898 56.134) (end 207.264 56.134) (width 0.25) (layer F.Cu) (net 2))
 (segment (start 199.898 56.134) (end 199.898 56.642) (width 0.25) (layer F.Cu) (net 2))
 (segment (start 199.898 56.134) (end 199.644 56.134) (width 0.25) (layer F.Cu) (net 2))
 (segment (start 199.644 56.134) (end 196.088 59.69) (width 0.25) (layer F.Cu) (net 2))
 (segment (start 196.088 59.69) (end 196.088 63.246) (width 0.25) (layer F.Cu) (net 2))
 (segment (start 172.948 62.992) (end 172.948 66.014) (width 0.25) (layer F.Cu) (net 5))
 (segment (start 172.948 66.014) (end 180.848 73.914) (width 0.25) (layer F.Cu) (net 5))
 (segment (start 188.748 66.014) (end 180.848 73.914) (width 0.25) (layer F.Cu) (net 5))
 (segment (start 188.748 62.992) (end 188.748 66.014) (width 0.25) (layer F.Cu) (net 5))
 (segment (start 183.633 99.06) (end 182.372 97.799) (width 0.25) (layer F.Cu) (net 5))
 (segment (start 184.658 99.06) (end 183.633 99.06) (width 0.25) (layer F.Cu) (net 5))
 (segment (start 182.372 97.799) (end 182.372 93.218) (width 0.25) (layer F.Cu) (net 5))
 (segment (start 182.372 93.218) (end 182.372 93.218) (width 0.25) (layer F.Cu) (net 5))
 (via (at 182.372 93.218) (size 0.8) (drill 0.4) (layers F.Cu B.Cu) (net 5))
 (via (at 180.847999 73.913999) (size 0.8) (drill 0.4) (layers F.Cu B.Cu) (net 5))
 (segment (start 182.372 93.218) (end 182.372 75.438) (width 0.25) (layer B.Cu) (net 5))
 (segment (start 182.372 75.438) (end 180.847999 73.913999) (width 0.25) (layer B.Cu) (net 5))
 (segment (start 180.848 73.914) (end 180.847999 73.913999) (width 0.25) (layer F.Cu) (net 5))
 (segment (start 172.974 96.52) (end 172.974 96.52) (width 0.25) (layer B.Cu) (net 9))
 (via (at 173.228 96.52) (size 0.8) (drill 0.4) (layers F.Cu B.Cu) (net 9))
 (segment (start 192.024 139.446) (end 185.166 139.446) (width 0.25) (layer B.Cu) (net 9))
 (segment (start 175.358 96.52) (end 173.228 96.52) (width 0.25) (layer F.Cu) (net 9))
 (segment (start 194.31 137.16) (end 192.024 139.446) (width 0.25) (layer B.Cu) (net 9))
 (segment (start 185.166 139.446) (end 168.402 122.682) (width 0.25) (layer B.Cu) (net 9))
 (segment (start 168.402 122.682) (end 168.402 98.044) (width 0.25) (layer B.Cu) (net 9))
 (segment (start 168.402 98.044) (end 169.926 96.52) (width 0.25) (layer B.Cu) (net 9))
 (segment (start 169.926 96.52) (end 173.228 96.52) (width 0.25) (layer B.Cu) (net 9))
 (via (at 173.228 101.34601) (size 0.8) (drill 0.4) (layers F.Cu B.Cu) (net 6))
 (segment (start 194.31 134.62) (end 189.992 130.302) (width 0.25) (layer B.Cu) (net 6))
 (segment (start 189.992 130.302) (end 189.992 118.11001) (width 0.25) (layer B.Cu) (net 6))
 (segment (start 189.992 118.11001) (end 173.228 101.34601) (width 0.25) (layer B.Cu) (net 6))
 (segment (start 175.358 100.33) (end 173.482 100.33) (width 0.25) (layer F.Cu) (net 6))
 (segment (start 173.228 100.584) (end 173.228 101.34601) (width 0.25) (layer F.Cu) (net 6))
 (segment (start 173.482 100.33) (end 173.228 100.584) (width 0.25) (layer F.Cu) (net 6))
 (segment (start 187.7425 97.79) (end 187.706 97.8265) (width 0.25) (layer F.Cu) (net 4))
 (segment (start 191.135 97.79) (end 187.7425 97.79) (width 0.25) (layer F.Cu) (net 4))
 (segment (start 184.6945 97.8265) (end 184.658 97.79) (width 0.25) (layer F.Cu) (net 4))
 (segment (start 187.706 97.8265) (end 184.6945 97.8265) (width 0.25) (layer F.Cu) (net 4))
 (segment (start 187.7425 95.25) (end 187.706 95.2135) (width 0.25) (layer F.Cu) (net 3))
 (segment (start 191.135 95.25) (end 187.7425 95.25) (width 0.25) (layer F.Cu) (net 3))
 (segment (start 185.9645 95.2135) (end 184.658 96.52) (width 0.25) (layer F.Cu) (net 3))
 (segment (start 187.706 95.2135) (end 185.9645 95.2135) (width 0.25) (layer F.Cu) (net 3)))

